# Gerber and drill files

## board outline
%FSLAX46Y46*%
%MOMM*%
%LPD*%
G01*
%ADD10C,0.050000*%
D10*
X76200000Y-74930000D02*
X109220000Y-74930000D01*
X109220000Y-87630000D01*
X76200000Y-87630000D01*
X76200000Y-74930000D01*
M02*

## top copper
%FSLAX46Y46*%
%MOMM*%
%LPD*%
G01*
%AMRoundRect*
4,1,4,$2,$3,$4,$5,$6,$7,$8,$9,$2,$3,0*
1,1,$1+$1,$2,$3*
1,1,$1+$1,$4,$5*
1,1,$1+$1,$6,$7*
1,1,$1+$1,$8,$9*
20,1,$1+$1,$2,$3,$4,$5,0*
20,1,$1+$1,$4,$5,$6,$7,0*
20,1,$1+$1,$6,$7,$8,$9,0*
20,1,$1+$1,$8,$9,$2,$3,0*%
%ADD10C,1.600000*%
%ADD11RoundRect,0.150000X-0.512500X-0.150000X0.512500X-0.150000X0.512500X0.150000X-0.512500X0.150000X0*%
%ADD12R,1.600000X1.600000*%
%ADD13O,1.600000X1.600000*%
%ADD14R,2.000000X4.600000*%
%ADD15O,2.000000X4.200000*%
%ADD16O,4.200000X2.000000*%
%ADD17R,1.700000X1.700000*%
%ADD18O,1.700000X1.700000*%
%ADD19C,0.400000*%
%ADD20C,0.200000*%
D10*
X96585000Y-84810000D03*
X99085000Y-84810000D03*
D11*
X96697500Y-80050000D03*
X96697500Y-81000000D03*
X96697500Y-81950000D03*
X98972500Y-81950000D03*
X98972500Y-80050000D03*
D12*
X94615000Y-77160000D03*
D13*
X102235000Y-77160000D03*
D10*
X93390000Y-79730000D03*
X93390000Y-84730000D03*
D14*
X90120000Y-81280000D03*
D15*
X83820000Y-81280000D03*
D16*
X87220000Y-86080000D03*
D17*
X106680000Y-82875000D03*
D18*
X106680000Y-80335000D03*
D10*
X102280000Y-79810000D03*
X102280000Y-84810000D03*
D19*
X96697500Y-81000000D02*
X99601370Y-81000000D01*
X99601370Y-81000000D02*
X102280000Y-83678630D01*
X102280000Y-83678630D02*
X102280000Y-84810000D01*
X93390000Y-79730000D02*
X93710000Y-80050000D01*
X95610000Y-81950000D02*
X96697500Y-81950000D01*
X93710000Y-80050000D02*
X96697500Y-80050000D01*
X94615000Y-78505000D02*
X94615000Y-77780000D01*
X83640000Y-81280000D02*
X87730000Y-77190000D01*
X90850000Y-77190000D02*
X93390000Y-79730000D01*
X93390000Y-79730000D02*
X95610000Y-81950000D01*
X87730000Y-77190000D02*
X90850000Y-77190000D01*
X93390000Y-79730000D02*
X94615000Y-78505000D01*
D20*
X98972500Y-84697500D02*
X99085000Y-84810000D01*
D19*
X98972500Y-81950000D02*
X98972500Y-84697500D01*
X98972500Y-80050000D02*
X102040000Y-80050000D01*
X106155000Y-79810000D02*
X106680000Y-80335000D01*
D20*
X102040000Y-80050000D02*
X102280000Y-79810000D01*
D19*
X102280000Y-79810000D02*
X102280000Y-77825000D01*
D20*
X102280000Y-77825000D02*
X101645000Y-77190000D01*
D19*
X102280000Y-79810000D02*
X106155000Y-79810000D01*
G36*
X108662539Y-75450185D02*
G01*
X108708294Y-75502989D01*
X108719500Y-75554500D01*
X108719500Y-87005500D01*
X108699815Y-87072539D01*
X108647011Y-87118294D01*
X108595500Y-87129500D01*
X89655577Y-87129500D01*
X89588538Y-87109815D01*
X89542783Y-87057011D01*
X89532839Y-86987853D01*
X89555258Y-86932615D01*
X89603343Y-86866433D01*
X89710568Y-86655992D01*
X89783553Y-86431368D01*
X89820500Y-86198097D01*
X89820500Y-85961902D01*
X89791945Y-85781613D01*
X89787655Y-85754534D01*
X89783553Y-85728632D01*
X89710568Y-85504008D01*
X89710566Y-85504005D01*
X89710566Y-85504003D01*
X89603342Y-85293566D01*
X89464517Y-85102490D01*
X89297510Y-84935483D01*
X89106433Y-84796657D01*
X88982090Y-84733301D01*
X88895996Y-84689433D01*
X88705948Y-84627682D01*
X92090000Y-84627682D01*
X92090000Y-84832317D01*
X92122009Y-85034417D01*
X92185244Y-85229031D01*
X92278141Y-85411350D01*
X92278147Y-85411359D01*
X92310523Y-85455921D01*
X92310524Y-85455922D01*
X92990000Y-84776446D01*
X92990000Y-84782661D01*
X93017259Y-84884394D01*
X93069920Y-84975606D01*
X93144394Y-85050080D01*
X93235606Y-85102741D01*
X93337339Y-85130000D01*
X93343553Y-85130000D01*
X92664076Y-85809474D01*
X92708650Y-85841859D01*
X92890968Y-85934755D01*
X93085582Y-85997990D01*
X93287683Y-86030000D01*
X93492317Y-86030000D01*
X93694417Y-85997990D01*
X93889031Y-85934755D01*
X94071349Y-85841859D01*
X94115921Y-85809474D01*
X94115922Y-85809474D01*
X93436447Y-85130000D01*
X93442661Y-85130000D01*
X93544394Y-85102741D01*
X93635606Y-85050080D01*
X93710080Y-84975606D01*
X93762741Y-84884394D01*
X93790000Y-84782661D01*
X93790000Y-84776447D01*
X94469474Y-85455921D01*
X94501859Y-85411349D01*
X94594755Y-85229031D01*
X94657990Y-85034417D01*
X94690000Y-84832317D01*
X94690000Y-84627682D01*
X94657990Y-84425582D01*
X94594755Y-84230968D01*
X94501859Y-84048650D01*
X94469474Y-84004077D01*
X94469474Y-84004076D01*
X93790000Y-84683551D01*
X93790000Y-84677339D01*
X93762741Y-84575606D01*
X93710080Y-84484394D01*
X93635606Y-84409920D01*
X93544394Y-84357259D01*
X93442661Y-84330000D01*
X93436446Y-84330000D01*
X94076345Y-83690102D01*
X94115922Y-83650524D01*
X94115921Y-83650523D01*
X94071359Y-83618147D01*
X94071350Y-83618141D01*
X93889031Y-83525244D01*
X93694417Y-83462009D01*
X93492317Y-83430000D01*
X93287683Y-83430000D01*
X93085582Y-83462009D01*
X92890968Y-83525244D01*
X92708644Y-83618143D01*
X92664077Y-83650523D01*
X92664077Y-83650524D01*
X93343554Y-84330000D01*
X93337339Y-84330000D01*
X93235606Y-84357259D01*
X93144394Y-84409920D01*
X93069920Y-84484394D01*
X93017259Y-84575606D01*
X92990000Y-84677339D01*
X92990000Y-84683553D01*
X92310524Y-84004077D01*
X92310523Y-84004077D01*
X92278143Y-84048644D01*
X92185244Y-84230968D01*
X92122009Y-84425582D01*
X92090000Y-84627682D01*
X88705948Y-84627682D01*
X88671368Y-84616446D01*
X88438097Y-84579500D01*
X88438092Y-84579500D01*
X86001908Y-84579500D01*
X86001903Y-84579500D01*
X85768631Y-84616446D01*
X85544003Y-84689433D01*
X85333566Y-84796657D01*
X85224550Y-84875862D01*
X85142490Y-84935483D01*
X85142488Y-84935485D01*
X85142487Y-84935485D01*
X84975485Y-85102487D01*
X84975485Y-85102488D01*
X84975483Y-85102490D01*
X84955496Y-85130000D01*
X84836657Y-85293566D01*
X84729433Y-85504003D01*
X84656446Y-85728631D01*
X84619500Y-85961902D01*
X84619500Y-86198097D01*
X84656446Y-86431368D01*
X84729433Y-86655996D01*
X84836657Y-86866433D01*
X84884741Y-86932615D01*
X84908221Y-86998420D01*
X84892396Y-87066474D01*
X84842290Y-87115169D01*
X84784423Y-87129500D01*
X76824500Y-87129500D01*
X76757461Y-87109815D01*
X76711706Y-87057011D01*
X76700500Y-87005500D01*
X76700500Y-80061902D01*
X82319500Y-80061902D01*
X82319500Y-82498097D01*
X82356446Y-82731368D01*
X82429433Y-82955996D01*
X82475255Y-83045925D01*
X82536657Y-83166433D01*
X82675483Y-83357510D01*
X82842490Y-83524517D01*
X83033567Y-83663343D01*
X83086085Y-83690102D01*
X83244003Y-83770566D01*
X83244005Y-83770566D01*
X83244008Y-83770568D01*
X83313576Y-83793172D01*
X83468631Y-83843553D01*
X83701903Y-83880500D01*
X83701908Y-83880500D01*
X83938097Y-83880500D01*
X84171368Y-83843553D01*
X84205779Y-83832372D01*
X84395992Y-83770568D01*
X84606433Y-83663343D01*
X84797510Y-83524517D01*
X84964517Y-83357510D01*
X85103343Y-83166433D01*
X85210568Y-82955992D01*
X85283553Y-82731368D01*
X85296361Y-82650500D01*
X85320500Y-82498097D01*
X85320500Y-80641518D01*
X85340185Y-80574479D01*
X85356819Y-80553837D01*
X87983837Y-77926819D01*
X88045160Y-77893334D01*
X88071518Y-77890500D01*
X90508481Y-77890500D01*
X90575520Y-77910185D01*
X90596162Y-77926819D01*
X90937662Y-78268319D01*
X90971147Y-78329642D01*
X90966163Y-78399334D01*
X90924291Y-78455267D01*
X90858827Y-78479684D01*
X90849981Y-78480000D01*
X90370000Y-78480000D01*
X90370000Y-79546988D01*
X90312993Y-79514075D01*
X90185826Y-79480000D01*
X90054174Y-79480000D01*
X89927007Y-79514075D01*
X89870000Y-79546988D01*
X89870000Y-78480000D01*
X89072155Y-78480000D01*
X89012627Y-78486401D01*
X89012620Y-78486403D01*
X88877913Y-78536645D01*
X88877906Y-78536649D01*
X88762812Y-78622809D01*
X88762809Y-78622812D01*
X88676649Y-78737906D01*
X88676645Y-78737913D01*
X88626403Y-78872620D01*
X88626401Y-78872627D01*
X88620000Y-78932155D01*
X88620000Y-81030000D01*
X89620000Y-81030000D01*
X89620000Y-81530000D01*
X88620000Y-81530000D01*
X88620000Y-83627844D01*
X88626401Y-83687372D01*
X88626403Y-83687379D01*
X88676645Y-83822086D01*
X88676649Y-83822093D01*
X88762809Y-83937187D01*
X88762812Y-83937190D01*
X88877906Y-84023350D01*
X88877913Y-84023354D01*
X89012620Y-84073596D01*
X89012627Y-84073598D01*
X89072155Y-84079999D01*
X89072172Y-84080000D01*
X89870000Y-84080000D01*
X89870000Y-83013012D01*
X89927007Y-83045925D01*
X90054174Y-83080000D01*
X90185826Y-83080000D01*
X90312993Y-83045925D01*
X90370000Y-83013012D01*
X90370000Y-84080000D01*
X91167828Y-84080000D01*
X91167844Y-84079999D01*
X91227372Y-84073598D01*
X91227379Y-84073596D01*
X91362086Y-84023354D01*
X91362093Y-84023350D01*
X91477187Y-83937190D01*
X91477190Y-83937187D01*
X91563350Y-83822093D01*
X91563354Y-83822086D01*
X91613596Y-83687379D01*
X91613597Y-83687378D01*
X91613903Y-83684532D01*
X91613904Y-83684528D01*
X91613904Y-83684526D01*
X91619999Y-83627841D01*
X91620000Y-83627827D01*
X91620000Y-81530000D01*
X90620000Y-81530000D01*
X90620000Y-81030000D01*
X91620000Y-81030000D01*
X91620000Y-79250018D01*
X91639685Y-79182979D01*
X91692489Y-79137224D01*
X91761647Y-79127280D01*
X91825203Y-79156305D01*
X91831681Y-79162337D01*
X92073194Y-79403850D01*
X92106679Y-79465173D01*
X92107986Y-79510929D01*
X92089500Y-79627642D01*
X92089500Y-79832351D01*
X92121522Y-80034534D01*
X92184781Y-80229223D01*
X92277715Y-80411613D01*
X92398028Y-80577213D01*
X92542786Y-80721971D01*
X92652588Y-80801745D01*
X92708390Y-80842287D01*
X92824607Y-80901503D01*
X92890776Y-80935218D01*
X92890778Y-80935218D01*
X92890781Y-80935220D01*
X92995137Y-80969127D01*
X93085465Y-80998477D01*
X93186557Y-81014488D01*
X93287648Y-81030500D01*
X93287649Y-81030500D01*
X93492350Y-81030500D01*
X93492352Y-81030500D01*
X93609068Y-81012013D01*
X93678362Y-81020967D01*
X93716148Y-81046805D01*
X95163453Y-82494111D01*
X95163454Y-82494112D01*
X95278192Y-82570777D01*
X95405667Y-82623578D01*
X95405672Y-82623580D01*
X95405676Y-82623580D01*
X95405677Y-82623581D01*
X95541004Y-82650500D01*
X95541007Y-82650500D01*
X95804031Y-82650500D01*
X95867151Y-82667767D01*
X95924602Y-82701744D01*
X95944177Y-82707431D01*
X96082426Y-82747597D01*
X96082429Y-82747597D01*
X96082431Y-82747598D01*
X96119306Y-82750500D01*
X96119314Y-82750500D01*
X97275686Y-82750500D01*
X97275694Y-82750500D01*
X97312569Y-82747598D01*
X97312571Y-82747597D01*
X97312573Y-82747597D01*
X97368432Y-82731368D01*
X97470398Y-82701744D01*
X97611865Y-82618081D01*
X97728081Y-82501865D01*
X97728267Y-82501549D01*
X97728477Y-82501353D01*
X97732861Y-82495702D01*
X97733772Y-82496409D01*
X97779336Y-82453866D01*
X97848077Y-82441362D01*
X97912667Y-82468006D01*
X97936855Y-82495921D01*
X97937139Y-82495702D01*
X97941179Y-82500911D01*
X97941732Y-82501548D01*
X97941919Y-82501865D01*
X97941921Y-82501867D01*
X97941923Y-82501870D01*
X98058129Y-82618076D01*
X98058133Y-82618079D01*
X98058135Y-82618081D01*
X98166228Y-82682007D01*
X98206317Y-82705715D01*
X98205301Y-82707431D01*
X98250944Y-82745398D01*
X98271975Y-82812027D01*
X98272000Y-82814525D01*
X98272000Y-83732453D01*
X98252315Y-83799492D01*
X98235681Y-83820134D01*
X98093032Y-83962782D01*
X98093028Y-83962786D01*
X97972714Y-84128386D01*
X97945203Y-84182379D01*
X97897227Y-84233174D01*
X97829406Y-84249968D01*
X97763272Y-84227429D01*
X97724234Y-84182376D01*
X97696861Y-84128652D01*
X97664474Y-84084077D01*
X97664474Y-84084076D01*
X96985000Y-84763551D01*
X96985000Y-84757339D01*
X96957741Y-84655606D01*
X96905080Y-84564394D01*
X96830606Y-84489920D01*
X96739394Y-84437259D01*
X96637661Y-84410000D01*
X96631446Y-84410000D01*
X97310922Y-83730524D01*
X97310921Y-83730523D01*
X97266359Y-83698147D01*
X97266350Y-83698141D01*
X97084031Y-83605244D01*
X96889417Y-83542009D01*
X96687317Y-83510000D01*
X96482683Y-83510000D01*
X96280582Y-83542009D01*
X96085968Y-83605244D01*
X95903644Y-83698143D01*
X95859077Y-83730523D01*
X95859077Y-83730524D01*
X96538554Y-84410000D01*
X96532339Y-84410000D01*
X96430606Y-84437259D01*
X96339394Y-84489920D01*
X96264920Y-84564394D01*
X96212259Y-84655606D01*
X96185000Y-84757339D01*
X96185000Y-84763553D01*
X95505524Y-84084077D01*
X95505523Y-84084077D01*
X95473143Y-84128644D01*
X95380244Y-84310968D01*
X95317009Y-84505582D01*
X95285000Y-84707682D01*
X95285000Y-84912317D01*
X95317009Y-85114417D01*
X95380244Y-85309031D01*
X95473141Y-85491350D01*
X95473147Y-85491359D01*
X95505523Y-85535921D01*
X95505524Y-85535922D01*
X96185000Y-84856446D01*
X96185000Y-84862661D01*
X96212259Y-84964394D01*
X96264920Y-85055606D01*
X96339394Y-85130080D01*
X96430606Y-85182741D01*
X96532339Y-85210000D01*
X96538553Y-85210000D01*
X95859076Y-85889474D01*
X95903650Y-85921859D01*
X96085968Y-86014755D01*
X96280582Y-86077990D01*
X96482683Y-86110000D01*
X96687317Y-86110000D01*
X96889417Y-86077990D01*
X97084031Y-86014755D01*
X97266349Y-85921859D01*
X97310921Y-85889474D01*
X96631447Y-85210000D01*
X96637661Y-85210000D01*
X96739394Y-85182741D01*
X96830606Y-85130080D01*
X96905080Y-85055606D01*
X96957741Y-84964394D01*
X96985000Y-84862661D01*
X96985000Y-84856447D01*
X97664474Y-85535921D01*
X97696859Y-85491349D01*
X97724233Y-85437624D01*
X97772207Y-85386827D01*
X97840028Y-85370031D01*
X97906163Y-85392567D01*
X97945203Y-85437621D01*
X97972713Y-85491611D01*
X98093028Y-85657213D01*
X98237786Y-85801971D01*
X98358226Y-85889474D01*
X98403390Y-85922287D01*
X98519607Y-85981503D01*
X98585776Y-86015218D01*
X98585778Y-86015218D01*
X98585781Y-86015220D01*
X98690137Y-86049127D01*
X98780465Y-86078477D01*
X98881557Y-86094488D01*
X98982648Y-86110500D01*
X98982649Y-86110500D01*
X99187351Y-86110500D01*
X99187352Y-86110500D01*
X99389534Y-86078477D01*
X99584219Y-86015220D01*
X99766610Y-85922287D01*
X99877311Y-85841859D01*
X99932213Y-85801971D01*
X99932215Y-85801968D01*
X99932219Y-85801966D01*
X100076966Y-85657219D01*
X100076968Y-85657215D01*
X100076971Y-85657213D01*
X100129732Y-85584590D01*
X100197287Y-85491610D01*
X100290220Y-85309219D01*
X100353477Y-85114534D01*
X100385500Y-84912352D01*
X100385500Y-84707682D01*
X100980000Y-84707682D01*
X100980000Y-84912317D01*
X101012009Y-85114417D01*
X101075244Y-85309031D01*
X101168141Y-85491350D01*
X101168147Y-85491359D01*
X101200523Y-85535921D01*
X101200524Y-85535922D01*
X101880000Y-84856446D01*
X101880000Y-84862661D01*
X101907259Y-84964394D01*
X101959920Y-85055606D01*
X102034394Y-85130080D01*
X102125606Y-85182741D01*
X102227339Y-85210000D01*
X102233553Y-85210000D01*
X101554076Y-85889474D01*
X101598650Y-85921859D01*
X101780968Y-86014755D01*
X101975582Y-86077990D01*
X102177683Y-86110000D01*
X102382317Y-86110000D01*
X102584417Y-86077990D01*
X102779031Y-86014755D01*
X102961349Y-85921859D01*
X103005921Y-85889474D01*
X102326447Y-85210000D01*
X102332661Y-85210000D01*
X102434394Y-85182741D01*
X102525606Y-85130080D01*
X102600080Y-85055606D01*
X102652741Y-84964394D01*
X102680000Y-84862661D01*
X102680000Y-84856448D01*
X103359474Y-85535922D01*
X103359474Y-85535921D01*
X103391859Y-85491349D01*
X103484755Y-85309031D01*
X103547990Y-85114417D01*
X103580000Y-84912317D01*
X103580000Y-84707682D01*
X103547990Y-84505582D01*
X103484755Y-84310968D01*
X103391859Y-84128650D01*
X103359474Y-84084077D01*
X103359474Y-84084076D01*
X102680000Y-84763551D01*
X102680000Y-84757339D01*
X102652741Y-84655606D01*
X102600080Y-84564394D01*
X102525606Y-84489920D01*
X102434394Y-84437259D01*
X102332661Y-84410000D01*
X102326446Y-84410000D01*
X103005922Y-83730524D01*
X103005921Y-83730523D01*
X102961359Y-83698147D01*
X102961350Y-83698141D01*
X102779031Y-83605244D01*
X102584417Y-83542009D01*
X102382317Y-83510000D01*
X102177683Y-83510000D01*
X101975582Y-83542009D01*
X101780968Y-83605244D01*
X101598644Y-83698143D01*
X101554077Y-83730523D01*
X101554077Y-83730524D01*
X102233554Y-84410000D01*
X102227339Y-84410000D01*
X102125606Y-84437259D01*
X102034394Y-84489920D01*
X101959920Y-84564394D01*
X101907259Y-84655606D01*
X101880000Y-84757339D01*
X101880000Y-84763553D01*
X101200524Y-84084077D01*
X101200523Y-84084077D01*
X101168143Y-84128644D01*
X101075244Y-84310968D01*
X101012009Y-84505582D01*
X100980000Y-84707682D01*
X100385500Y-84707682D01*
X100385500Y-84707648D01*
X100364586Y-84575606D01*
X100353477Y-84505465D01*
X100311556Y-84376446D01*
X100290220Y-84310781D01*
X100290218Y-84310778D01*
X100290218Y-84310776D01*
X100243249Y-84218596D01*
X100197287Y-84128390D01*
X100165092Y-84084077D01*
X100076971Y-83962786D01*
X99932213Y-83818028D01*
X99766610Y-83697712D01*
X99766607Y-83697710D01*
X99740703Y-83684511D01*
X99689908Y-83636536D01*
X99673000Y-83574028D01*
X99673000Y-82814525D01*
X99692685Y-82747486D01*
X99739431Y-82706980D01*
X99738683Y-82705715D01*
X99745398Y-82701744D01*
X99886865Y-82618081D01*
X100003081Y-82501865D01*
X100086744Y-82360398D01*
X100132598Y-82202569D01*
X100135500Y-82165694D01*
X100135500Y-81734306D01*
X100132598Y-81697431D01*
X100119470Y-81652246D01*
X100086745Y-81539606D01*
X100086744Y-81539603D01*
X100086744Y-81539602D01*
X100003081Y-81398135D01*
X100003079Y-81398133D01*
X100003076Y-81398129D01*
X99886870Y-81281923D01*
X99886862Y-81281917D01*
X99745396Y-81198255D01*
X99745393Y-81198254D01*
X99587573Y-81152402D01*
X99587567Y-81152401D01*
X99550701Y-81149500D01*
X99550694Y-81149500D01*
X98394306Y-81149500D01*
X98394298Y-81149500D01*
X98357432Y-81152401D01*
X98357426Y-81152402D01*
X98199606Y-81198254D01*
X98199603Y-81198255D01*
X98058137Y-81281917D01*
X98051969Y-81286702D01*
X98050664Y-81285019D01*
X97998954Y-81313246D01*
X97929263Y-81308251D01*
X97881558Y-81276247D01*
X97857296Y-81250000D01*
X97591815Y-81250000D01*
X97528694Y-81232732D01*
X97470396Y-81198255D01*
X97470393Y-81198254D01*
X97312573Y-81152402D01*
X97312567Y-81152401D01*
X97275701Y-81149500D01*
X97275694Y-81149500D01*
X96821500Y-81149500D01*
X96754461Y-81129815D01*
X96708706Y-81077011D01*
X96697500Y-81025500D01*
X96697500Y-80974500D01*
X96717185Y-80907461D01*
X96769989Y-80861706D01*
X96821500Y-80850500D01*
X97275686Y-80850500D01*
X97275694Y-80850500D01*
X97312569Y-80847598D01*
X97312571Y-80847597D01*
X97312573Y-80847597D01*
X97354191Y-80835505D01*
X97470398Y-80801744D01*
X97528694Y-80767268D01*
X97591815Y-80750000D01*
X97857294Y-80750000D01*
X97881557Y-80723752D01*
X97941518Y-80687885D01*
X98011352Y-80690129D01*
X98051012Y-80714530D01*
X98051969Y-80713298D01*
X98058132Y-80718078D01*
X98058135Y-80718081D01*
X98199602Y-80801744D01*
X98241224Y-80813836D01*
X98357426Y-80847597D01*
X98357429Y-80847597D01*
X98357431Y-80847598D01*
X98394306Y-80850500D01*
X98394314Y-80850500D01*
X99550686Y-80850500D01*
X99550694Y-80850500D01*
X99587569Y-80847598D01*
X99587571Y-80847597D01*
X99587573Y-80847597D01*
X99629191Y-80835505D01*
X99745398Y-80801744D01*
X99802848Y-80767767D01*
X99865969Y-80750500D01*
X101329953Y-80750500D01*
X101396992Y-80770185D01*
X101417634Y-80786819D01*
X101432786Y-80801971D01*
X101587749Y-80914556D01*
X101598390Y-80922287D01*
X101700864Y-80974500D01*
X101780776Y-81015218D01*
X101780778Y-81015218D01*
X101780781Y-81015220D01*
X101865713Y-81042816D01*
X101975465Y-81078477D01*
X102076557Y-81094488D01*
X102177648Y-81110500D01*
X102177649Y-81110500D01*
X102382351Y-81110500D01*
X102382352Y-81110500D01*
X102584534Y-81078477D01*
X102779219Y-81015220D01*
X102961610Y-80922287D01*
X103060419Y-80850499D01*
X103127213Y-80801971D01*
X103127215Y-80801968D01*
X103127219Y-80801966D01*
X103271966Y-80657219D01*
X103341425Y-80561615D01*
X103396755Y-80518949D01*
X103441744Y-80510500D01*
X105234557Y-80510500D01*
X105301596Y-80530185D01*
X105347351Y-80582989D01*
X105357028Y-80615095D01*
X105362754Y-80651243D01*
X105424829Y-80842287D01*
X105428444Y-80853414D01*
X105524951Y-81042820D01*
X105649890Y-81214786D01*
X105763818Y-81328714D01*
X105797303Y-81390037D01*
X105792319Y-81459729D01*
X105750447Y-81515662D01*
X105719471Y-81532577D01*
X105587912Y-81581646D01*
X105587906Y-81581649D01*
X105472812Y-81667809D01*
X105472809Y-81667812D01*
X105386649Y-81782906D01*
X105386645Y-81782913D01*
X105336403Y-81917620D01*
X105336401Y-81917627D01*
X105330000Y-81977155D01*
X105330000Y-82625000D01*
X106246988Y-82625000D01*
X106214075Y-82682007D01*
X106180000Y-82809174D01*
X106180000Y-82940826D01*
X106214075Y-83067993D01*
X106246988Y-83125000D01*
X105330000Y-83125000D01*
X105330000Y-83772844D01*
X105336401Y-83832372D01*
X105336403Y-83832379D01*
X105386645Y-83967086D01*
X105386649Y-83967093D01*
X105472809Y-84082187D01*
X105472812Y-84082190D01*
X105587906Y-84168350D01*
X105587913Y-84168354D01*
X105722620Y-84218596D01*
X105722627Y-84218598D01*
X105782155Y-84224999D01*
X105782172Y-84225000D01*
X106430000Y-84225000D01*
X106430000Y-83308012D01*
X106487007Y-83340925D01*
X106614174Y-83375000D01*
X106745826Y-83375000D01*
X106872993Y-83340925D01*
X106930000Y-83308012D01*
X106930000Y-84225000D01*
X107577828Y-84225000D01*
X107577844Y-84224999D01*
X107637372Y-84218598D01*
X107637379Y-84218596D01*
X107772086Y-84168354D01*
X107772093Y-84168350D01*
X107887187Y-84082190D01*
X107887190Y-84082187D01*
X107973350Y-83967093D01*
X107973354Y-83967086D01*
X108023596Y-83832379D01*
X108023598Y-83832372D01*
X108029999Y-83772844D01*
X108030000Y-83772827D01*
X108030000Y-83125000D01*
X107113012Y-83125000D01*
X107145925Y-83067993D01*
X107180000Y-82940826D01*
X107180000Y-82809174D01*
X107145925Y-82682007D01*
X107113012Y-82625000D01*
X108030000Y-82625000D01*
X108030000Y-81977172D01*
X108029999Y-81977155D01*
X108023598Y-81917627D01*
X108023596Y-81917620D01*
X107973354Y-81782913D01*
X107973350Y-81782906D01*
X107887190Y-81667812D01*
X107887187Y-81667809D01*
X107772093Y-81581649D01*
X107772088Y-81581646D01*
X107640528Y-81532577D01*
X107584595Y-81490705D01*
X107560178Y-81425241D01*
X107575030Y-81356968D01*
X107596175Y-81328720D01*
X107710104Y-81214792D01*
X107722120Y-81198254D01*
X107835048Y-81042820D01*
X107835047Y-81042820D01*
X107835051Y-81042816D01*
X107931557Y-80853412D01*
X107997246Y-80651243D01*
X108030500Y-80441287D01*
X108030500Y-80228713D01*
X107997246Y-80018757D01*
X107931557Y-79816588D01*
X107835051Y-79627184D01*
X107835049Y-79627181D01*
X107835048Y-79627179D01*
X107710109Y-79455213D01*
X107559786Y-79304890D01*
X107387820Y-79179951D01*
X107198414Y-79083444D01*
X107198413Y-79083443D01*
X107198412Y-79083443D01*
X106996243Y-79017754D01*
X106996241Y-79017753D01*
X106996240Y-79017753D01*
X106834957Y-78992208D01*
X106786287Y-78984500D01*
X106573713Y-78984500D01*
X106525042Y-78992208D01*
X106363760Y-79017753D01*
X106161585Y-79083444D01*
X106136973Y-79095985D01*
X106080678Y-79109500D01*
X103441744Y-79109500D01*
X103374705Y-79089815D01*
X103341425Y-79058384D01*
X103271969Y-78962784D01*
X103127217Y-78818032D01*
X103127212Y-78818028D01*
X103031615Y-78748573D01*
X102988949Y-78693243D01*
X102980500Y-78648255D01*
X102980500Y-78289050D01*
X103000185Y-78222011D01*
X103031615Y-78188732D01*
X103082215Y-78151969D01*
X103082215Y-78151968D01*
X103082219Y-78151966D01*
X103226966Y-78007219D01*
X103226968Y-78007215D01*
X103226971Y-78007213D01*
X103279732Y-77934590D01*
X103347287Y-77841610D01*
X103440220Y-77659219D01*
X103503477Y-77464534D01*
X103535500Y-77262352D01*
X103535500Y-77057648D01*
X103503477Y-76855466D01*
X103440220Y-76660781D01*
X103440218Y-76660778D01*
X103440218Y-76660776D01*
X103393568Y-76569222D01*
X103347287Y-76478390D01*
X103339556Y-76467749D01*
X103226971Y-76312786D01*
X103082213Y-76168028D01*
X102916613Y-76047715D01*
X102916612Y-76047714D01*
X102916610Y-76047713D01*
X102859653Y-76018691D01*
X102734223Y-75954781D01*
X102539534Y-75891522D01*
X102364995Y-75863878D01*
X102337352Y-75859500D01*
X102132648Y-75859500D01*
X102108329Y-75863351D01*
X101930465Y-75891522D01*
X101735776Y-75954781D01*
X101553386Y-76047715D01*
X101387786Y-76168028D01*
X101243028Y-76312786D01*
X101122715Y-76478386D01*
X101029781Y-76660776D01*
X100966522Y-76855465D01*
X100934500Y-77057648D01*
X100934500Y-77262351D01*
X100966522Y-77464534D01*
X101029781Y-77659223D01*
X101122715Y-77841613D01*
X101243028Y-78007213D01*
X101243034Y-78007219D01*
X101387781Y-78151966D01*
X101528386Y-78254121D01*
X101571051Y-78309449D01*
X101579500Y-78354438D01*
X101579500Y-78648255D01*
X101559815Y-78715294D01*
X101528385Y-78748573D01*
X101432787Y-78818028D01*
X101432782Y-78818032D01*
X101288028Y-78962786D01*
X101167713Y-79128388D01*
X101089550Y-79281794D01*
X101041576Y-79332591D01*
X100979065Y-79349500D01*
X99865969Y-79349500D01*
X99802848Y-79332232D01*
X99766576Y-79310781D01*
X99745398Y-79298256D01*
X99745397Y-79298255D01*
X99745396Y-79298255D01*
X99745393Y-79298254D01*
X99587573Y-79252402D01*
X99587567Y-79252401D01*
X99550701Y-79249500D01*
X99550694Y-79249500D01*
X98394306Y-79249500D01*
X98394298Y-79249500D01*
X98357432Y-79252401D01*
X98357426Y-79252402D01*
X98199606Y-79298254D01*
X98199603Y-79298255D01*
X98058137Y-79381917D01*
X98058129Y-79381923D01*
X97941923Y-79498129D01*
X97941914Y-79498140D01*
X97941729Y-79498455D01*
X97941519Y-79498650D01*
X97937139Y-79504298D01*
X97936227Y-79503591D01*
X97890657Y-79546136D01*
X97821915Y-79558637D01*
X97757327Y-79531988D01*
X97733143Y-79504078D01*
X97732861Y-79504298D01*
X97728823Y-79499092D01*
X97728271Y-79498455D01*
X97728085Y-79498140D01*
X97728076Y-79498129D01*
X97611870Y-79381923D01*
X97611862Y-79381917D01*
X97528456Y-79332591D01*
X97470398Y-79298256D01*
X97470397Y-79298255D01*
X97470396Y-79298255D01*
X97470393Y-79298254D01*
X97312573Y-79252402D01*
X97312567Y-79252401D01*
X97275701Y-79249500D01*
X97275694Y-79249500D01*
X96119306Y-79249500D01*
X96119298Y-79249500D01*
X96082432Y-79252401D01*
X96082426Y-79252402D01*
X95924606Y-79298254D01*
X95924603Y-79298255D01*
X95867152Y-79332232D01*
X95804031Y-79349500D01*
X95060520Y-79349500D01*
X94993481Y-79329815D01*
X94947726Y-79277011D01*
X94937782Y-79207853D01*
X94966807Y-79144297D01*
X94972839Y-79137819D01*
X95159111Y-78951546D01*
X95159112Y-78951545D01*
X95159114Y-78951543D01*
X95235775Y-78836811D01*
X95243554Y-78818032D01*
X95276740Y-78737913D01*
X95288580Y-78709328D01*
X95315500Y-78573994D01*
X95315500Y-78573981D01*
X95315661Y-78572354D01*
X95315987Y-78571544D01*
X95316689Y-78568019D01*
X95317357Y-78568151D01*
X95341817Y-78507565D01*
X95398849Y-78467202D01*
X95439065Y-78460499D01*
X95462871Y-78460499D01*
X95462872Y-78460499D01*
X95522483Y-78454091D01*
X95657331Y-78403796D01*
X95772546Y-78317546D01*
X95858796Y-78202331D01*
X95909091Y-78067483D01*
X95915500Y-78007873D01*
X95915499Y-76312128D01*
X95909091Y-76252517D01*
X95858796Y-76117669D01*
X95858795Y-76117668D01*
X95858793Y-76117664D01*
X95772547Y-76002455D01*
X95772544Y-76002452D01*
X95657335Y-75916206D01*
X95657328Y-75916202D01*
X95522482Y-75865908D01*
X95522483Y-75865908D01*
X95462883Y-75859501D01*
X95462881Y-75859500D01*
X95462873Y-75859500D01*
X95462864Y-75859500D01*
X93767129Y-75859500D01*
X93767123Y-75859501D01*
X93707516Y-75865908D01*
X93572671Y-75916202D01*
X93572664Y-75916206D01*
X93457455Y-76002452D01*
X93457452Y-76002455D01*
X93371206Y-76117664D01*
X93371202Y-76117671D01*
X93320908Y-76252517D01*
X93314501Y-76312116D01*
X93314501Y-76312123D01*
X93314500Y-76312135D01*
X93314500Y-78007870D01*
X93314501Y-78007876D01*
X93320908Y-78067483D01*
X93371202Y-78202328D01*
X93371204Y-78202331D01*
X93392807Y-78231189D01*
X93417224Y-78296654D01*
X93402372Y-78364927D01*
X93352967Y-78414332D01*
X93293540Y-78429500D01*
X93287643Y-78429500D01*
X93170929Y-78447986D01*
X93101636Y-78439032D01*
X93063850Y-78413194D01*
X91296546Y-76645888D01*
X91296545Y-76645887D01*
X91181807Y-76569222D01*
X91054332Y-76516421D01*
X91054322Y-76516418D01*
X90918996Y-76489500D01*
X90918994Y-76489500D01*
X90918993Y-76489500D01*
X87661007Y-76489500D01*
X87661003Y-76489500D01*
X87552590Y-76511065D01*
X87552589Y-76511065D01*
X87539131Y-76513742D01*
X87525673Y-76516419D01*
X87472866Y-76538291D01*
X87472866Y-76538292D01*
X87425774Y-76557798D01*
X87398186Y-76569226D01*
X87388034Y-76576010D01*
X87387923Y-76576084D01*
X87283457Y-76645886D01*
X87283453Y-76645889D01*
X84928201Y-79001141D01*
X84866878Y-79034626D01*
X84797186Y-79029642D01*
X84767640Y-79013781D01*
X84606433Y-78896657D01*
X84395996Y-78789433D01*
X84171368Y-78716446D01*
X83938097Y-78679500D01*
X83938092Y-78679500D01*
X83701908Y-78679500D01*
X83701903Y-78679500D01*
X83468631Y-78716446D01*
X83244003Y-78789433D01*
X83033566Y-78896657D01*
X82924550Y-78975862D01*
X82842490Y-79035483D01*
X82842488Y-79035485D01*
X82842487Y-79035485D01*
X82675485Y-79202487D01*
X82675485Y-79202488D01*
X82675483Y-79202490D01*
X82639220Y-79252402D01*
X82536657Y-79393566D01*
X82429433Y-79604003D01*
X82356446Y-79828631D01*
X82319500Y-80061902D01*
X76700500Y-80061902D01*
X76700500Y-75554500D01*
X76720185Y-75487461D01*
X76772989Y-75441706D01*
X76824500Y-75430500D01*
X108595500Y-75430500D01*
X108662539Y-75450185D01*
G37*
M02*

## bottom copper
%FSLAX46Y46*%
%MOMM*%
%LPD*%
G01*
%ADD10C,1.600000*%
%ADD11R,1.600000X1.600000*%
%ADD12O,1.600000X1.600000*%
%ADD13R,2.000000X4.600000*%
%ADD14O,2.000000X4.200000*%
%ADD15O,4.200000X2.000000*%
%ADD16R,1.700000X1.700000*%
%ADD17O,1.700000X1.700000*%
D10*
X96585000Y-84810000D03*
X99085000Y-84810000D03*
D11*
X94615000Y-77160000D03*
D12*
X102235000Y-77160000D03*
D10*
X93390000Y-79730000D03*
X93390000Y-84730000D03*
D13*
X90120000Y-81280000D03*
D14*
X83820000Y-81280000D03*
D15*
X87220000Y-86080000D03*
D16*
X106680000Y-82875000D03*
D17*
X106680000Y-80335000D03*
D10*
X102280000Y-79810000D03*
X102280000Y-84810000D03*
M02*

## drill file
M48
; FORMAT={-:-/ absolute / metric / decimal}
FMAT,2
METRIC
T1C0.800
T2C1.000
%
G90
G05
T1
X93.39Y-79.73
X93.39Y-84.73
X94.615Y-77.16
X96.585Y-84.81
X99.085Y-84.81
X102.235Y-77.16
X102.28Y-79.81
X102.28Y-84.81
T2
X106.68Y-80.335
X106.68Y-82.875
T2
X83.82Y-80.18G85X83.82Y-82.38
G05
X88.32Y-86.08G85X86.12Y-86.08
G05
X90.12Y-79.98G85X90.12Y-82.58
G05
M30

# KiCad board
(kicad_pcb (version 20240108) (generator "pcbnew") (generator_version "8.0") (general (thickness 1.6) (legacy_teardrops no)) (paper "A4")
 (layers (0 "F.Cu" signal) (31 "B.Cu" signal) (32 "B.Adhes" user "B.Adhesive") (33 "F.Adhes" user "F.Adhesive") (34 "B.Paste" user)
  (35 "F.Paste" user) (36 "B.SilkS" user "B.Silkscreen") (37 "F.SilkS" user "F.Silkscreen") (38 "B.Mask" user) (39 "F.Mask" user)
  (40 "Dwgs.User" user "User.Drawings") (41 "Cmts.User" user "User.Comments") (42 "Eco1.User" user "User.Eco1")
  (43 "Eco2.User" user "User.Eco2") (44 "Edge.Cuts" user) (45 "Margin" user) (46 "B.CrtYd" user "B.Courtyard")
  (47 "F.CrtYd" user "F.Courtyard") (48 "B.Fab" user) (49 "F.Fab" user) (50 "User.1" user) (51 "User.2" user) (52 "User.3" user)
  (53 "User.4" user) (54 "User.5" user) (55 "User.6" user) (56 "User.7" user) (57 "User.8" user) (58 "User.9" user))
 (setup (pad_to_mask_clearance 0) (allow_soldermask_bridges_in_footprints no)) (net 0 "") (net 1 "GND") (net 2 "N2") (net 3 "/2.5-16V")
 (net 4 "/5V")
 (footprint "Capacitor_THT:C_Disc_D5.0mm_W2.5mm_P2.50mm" (layer "F.Cu") (at 96.585 84.81)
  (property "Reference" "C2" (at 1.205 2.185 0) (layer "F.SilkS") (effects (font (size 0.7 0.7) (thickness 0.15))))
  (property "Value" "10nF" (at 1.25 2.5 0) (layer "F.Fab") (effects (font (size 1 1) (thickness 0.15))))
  (pad "1" thru_hole circle (at 0 0) (size 1.6 1.6) (drill 0.8) (layers "*.Cu" "*.Mask") (remove_unused_layers no) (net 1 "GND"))
  (pad "2" thru_hole circle (at 2.5 0) (size 1.6 1.6) (drill 0.8) (layers "*.Cu" "*.Mask") (remove_unused_layers no) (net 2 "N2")))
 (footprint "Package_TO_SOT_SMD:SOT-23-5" (layer "F.Cu") (at 97.835 81)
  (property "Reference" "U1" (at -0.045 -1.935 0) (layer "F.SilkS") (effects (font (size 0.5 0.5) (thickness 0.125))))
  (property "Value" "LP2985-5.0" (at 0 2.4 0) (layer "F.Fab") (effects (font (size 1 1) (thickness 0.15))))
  (pad "1" smd roundrect (at -1.1375 -0.95) (size 1.325 0.6) (layers "F.Cu" "F.Paste" "F.Mask") (roundrect_rratio 0.25) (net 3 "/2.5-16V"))
  (pad "2" smd roundrect (at -1.1375 0) (size 1.325 0.6) (layers "F.Cu" "F.Paste" "F.Mask") (roundrect_rratio 0.25) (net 1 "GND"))
  (pad "3" smd roundrect (at -1.1375 0.95) (size 1.325 0.6) (layers "F.Cu" "F.Paste" "F.Mask") (roundrect_rratio 0.25) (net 3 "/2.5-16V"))
  (pad "4" smd roundrect (at 1.1375 0.95) (size 1.325 0.6) (layers "F.Cu" "F.Paste" "F.Mask") (roundrect_rratio 0.25) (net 2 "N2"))
  (pad "5" smd roundrect (at 1.1375 -0.95) (size 1.325 0.6) (layers "F.Cu" "F.Paste" "F.Mask") (roundrect_rratio 0.25) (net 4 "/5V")))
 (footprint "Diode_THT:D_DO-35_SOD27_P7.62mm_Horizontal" (layer "F.Cu") (at 94.615 77.16)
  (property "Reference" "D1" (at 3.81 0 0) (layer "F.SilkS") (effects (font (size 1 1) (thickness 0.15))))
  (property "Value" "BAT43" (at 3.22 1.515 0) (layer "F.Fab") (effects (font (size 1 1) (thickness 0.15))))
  (pad "1" thru_hole rect (at 0 0) (size 1.6 1.6) (drill 0.8) (layers "*.Cu" "*.Mask") (remove_unused_layers no) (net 3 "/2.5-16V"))
  (pad "2" thru_hole oval (at 7.62 0) (size 1.6 1.6) (drill 0.8) (layers "*.Cu" "*.Mask") (remove_unused_layers no) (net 4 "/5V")))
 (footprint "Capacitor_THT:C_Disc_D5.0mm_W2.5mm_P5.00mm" (layer "F.Cu") (at 93.39 79.73 -90)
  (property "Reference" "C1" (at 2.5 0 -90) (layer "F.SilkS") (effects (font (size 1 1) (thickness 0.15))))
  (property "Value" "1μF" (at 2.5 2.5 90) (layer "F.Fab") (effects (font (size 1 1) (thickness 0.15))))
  (pad "1" thru_hole circle (at 0 0 270) (size 1.6 1.6) (drill 0.8) (layers "*.Cu" "*.Mask") (remove_unused_layers no) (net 3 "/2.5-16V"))
  (pad "2" thru_hole circle (at 5 0 270) (size 1.6 1.6) (drill 0.8) (layers "*.Cu" "*.Mask") (remove_unused_layers no) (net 1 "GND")))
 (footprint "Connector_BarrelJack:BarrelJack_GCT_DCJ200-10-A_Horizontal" (layer "F.Cu") (at 90.12 81.28 -90)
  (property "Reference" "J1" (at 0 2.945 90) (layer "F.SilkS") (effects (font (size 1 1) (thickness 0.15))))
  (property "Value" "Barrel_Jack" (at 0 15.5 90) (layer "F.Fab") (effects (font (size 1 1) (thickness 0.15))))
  (pad "1" thru_hole rect (at 0 0 270) (size 4.6 2) (drill oval 3.6 1) (layers "*.Cu" "*.Mask") (remove_unused_layers no) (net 1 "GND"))
  (pad "2" thru_hole oval (at 0 6.3 270) (size 4.2 2) (drill oval 3.2 1) (layers "*.Cu" "*.Mask") (remove_unused_layers no)
   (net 3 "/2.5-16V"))
  (pad "3" thru_hole oval (at 4.8 2.9 270) (size 2 4.2) (drill oval 1 3.2) (layers "*.Cu" "*.Mask") (remove_unused_layers no)))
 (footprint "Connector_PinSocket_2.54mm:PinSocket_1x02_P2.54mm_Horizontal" (layer "F.Cu") (at 106.68 82.875 180)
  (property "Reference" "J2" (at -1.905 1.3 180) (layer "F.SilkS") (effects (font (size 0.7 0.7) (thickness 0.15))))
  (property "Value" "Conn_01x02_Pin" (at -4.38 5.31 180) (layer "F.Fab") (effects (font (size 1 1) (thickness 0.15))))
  (pad "1" thru_hole rect (at 0 0 180) (size 1.7 1.7) (drill 1) (layers "*.Cu" "*.Mask") (remove_unused_layers no) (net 1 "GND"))
  (pad "2" thru_hole oval (at 0 2.54 180) (size 1.7 1.7) (drill 1) (layers "*.Cu" "*.Mask") (remove_unused_layers no) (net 4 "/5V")))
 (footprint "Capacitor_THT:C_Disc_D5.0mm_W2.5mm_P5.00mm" (layer "F.Cu") (at 102.28 79.81 -90)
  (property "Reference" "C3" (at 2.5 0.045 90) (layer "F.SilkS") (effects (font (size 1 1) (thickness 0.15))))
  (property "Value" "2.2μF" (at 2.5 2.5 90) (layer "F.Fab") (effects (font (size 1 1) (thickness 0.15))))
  (pad "1" thru_hole circle (at 0 0 270) (size 1.6 1.6) (drill 0.8) (layers "*.Cu" "*.Mask") (remove_unused_layers no) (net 4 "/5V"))
  (pad "2" thru_hole circle (at 5 0 270) (size 1.6 1.6) (drill 0.8) (layers "*.Cu" "*.Mask") (remove_unused_layers no) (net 1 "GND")))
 (gr_rect (start 76.2 74.93) (end 109.22 87.63) (stroke (width 0.05) (type default)) (fill none) (layer "Edge.Cuts"))
 (segment (start 96.6975 81) (end 99.60137 81) (width 0.4) (layer "F.Cu") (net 1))
 (segment (start 99.60137 81) (end 102.28 83.67863) (width 0.4) (layer "F.Cu") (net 1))
 (segment (start 102.28 83.67863) (end 102.28 84.81) (width 0.4) (layer "F.Cu") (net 1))
 (segment (start 93.39 79.73) (end 93.71 80.05) (width 0.4) (layer "F.Cu") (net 3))
 (segment (start 95.61 81.95) (end 96.6975 81.95) (width 0.4) (layer "F.Cu") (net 3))
 (segment (start 93.71 80.05) (end 96.6975 80.05) (width 0.4) (layer "F.Cu") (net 3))
 (segment (start 94.615 78.505) (end 94.615 77.78) (width 0.4) (layer "F.Cu") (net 3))
 (segment (start 83.64 81.28) (end 87.73 77.19) (width 0.4) (layer "F.Cu") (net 3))
 (segment (start 90.85 77.19) (end 93.39 79.73) (width 0.4) (layer "F.Cu") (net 3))
 (segment (start 93.39 79.73) (end 95.61 81.95) (width 0.4) (layer "F.Cu") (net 3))
 (segment (start 87.73 77.19) (end 90.85 77.19) (width 0.4) (layer "F.Cu") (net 3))
 (segment (start 93.39 79.73) (end 94.615 78.505) (width 0.4) (layer "F.Cu") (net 3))
 (segment (start 98.9725 84.6975) (end 99.085 84.81) (width 0.2) (layer "F.Cu") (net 2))
 (segment (start 98.9725 81.95) (end 98.9725 84.6975) (width 0.4) (layer "F.Cu") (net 2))
 (segment (start 98.9725 80.05) (end 102.04 80.05) (width 0.4) (layer "F.Cu") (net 4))
 (segment (start 106.155 79.81) (end 106.68 80.335) (width 0.4) (layer "F.Cu") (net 4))
 (segment (start 102.04 80.05) (end 102.28 79.81) (width 0.2) (layer "F.Cu") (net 4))
 (segment (start 102.28 79.81) (end 102.28 77.825) (width 0.4) (layer "F.Cu") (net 4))
 (segment (start 102.28 77.825) (end 101.645 77.19) (width 0.2) (layer "F.Cu") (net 4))
 (segment (start 102.28 79.81) (end 106.155 79.81) (width 0.4) (layer "F.Cu") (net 4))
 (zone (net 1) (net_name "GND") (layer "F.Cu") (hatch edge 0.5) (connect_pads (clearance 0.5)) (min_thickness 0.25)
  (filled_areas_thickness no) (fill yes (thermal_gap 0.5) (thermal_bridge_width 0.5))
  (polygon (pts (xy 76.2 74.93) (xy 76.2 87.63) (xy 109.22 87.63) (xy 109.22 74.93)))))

